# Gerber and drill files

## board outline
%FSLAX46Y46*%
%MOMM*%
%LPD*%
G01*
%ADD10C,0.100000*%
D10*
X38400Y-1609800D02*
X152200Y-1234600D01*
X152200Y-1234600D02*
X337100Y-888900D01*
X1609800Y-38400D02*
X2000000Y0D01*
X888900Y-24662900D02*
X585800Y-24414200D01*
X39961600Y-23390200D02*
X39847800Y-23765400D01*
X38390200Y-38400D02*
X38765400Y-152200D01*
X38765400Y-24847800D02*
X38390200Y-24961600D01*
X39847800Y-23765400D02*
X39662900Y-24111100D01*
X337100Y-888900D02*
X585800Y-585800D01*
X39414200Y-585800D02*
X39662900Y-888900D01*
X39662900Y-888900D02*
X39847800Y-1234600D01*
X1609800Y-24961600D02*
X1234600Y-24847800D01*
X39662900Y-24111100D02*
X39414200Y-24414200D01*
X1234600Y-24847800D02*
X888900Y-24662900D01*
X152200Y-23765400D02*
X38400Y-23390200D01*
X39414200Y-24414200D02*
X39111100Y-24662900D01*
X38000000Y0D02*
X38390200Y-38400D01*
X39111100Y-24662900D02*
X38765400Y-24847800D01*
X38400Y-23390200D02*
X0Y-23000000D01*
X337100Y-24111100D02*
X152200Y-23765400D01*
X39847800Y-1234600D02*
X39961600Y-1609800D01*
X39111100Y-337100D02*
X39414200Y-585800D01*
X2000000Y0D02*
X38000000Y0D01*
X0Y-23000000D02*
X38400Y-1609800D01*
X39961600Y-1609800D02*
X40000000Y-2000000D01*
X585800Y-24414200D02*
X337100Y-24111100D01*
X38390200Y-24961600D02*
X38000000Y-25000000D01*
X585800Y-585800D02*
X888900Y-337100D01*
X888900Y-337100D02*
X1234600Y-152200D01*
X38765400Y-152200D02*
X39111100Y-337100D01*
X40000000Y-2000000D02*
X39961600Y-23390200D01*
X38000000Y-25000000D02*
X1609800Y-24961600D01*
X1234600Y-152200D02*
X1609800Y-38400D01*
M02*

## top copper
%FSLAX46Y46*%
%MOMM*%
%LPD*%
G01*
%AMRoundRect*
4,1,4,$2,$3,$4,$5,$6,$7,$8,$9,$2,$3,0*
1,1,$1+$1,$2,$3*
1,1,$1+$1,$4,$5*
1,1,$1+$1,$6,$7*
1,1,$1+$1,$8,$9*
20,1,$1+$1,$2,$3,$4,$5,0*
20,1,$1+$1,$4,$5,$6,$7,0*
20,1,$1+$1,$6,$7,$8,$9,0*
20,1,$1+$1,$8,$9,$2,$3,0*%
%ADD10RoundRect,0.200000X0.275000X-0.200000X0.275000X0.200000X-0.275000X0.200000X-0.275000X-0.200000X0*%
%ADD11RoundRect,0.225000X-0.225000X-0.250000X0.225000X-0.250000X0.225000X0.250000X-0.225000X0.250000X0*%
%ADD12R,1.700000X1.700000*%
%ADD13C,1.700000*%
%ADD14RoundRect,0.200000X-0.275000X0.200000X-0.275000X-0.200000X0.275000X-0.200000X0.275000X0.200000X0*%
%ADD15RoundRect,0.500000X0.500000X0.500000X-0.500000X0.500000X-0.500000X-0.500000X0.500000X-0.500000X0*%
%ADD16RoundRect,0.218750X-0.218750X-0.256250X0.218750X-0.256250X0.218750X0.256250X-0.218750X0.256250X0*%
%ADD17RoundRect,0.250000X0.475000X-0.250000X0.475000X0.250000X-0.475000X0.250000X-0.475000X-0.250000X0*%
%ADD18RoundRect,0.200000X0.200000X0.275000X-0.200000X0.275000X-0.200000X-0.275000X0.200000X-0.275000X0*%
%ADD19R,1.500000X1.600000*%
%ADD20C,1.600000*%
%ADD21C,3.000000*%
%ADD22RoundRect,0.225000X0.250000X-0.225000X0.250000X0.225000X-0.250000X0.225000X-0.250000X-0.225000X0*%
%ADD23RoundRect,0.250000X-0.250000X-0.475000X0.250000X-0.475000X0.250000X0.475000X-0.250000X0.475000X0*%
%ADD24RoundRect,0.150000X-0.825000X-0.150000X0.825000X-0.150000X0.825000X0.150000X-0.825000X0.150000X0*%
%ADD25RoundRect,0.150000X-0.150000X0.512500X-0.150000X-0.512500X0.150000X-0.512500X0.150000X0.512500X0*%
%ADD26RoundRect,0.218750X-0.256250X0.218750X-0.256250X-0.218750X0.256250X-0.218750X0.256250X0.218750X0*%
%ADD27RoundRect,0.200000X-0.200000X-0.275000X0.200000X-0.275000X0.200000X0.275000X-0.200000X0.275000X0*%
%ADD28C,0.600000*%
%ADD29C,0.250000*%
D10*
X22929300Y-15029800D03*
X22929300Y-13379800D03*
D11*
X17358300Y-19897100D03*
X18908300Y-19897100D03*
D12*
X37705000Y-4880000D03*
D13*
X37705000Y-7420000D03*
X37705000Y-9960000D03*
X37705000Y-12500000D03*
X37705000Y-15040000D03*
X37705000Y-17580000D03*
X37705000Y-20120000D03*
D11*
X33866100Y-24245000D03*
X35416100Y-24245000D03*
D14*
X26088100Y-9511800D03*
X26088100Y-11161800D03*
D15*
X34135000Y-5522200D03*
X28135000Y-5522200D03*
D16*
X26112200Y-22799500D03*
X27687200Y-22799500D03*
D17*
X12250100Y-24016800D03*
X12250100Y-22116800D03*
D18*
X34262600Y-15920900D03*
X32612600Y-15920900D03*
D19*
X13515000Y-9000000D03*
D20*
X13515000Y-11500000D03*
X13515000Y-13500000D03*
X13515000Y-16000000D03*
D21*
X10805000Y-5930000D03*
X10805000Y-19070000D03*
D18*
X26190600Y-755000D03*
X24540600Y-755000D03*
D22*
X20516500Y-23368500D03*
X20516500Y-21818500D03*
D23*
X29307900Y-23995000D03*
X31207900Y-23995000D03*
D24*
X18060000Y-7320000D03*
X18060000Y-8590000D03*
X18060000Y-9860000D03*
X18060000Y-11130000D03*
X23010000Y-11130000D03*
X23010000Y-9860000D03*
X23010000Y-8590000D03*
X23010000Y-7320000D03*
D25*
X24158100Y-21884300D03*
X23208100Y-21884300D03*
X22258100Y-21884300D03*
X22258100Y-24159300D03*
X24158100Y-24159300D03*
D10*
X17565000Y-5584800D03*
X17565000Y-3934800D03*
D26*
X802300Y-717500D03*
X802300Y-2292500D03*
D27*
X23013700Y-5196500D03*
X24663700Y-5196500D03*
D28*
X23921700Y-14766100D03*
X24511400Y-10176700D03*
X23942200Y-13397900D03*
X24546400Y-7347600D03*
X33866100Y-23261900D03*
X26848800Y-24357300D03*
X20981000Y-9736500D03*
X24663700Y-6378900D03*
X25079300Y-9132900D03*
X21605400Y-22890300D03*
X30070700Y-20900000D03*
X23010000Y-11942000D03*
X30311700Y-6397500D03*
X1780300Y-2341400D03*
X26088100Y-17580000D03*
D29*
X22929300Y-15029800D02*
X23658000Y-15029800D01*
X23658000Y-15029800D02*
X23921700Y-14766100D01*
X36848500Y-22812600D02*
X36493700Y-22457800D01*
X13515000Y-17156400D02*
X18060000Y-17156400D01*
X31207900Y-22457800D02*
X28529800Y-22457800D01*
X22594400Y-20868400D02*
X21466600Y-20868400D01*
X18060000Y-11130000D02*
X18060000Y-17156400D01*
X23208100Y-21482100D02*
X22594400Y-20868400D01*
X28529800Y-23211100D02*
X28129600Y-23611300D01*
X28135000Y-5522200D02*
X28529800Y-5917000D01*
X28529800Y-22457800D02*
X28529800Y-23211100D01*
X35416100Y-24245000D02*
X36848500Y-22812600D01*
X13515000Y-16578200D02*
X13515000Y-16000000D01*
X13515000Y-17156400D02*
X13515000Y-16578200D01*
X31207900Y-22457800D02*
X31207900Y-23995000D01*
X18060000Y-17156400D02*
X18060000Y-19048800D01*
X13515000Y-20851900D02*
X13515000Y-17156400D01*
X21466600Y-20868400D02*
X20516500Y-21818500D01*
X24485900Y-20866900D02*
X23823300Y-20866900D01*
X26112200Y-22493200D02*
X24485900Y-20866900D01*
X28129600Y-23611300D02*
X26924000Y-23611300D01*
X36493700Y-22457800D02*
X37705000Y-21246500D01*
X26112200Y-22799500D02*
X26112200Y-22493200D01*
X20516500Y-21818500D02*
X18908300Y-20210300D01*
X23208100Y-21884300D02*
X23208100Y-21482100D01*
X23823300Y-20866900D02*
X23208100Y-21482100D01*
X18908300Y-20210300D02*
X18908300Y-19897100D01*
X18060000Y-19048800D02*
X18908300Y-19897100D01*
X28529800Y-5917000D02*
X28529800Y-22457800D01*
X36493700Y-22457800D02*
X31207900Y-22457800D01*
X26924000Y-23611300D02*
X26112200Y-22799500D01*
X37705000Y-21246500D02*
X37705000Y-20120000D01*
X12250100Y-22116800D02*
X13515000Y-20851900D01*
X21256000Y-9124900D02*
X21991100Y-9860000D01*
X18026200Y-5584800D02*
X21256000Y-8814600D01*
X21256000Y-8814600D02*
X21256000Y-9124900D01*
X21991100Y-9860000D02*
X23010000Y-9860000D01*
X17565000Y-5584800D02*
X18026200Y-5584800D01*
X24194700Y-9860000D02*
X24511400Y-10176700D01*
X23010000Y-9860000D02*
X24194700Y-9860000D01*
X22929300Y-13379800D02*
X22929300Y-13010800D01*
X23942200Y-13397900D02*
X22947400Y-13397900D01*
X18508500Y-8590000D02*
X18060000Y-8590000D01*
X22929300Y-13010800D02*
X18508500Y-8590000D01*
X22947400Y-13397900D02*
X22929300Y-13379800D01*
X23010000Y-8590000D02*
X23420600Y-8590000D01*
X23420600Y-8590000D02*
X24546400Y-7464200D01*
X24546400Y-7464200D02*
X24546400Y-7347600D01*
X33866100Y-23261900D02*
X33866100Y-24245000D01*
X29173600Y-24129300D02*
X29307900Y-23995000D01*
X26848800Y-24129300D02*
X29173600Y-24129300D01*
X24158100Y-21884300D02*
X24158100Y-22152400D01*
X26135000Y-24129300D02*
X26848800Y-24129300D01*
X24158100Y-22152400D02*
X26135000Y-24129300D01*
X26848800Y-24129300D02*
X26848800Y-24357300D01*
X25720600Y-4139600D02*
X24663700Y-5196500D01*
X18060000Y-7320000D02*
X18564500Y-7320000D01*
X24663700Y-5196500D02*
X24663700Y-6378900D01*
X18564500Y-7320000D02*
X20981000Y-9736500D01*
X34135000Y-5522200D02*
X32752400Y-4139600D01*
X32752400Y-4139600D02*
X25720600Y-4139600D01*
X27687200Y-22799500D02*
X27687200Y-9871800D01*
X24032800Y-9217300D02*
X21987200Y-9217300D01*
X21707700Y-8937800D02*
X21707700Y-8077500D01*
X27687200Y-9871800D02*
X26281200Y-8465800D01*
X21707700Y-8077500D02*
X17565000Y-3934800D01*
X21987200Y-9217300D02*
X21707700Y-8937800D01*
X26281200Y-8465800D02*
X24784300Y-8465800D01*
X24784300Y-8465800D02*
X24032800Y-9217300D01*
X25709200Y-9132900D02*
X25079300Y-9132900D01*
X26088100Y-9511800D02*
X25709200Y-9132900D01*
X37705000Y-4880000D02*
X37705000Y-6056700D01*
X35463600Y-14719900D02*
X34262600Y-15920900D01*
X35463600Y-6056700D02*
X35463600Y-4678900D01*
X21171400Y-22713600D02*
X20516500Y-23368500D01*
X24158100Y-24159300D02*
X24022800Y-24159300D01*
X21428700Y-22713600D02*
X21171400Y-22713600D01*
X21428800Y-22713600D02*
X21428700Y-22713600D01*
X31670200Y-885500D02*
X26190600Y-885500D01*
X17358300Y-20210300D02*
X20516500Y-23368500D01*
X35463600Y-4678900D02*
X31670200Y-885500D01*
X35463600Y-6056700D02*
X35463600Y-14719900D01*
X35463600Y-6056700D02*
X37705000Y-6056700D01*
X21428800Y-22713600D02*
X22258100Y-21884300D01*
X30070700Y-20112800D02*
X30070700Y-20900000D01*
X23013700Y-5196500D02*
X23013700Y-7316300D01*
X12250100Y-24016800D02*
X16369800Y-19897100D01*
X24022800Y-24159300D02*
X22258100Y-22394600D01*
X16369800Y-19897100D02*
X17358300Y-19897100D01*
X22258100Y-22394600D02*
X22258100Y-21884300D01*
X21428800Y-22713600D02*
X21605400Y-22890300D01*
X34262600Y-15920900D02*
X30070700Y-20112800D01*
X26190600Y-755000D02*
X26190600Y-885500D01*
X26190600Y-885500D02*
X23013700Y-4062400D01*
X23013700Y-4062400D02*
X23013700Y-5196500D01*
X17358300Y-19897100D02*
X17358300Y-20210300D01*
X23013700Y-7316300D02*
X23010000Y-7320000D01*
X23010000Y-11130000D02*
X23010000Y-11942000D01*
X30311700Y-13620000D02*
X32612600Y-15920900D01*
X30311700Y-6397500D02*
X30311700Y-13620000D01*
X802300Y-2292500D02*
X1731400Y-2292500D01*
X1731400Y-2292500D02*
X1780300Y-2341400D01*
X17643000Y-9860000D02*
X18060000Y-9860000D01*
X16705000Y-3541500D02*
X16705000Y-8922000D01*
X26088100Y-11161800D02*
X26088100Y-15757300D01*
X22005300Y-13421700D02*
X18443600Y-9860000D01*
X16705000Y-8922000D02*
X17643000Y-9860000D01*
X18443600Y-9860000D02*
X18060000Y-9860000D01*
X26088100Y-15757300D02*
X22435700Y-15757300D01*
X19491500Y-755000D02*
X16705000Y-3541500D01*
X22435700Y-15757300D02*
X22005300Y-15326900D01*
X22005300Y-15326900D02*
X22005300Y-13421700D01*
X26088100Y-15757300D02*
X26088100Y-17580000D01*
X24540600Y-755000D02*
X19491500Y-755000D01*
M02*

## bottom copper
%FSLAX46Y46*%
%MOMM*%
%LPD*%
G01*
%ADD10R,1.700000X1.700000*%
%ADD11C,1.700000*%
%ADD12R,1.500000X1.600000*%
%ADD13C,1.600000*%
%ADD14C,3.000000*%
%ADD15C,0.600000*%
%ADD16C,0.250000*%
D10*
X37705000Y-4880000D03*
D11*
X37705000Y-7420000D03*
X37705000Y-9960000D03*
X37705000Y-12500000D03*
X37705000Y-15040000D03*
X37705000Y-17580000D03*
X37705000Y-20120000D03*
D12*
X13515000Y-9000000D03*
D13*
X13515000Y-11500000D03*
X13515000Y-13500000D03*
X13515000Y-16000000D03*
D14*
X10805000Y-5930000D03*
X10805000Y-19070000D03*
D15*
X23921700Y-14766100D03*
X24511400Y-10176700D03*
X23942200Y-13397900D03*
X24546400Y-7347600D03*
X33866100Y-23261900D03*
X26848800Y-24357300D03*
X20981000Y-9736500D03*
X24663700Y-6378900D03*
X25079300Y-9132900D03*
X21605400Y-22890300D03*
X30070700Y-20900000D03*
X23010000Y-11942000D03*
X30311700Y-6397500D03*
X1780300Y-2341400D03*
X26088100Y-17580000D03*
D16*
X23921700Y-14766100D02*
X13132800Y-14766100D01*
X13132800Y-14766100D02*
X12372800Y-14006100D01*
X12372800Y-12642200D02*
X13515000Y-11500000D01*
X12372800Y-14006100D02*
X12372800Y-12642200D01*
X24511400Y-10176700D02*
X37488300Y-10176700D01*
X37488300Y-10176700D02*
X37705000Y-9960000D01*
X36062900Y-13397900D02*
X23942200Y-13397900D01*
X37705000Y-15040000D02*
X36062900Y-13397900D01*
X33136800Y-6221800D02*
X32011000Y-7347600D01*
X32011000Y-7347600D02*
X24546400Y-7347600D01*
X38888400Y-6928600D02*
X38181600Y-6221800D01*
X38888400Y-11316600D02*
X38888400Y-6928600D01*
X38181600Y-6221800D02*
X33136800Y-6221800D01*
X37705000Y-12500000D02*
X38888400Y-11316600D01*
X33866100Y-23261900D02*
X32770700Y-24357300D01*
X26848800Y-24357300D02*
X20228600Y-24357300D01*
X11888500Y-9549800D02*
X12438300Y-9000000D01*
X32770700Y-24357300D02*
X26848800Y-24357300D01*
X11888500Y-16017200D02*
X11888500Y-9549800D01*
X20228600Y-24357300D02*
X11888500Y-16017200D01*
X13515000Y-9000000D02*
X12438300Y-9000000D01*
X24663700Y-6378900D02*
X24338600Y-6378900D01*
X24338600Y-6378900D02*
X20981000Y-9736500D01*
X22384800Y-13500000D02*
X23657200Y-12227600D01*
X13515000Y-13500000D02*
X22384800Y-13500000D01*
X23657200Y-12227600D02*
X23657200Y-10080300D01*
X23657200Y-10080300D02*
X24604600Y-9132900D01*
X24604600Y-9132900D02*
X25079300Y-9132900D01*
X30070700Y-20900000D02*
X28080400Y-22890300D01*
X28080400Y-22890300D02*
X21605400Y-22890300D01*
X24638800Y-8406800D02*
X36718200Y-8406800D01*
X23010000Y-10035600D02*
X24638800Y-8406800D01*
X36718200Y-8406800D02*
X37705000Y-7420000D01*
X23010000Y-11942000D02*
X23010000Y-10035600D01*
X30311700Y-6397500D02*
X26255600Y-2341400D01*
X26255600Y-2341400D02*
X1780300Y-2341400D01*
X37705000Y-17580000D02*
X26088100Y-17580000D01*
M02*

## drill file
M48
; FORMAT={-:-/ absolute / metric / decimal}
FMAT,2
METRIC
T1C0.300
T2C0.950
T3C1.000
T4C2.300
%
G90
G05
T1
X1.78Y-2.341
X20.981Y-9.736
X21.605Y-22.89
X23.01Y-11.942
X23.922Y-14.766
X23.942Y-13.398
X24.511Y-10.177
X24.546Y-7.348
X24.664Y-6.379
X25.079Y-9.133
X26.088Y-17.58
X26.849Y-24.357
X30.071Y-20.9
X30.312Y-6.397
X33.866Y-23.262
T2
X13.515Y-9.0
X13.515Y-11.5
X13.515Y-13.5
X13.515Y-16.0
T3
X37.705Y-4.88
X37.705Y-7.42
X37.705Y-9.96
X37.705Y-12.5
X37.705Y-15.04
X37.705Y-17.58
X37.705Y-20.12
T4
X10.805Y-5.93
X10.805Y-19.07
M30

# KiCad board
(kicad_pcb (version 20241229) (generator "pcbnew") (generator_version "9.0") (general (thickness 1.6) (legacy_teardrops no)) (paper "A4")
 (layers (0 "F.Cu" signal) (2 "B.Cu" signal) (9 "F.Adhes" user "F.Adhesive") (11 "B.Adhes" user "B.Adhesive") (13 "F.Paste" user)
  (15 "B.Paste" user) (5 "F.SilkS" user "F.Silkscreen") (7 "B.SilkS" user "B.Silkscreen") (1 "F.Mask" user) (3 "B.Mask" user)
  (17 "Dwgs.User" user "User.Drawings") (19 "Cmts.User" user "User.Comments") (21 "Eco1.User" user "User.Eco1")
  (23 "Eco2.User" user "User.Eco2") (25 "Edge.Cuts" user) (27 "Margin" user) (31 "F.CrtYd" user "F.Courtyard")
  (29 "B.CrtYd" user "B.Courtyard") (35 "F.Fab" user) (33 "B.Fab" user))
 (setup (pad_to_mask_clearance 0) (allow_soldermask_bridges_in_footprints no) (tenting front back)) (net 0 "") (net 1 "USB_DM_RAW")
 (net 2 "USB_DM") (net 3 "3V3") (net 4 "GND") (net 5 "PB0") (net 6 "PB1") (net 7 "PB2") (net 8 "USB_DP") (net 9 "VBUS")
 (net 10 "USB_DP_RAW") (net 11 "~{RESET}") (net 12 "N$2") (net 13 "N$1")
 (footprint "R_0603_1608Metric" (layer "F.Cu") (at 22.9293 14.2048 90)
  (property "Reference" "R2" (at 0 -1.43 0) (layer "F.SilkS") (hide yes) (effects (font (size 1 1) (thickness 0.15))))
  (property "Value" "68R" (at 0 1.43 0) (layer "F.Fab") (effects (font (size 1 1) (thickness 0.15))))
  (pad "1" smd roundrect (at -0.825 0 90) (size 0.8 0.95) (layers "F.Cu" "F.Mask" "F.Paste") (roundrect_rratio 0.25) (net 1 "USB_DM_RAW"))
  (pad "2" smd roundrect (at 0.825 0 90) (size 0.8 0.95) (layers "F.Cu" "F.Mask" "F.Paste") (roundrect_rratio 0.25) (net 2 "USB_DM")))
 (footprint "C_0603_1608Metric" (layer "F.Cu") (at 18.1333 19.8971)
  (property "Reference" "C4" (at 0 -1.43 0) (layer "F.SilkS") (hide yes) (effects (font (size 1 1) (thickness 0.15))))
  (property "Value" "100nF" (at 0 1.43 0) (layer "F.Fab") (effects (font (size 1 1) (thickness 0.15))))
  (pad "1" smd roundrect (at -0.775 0) (size 0.9 0.95) (layers "F.Cu" "F.Mask" "F.Paste") (roundrect_rratio 0.25) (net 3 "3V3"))
  (pad "2" smd roundrect (at 0.775 0) (size 0.9 0.95) (layers "F.Cu" "F.Mask" "F.Paste") (roundrect_rratio 0.25) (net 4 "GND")))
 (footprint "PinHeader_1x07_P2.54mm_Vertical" (layer "F.Cu") (at 37.705 4.88)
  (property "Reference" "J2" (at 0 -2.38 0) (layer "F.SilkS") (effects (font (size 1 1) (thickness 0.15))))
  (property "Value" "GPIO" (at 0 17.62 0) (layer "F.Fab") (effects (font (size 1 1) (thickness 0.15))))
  (pad "1" thru_hole rect (at 0 0) (size 1.7 1.7) (drill 1) (layers "*.Cu" "*.Mask") (remove_unused_layers no) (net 3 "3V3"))
  (pad "2" thru_hole circle (at 0 2.54) (size 1.7 1.7) (drill 1) (layers "*.Cu" "*.Mask") (remove_unused_layers no) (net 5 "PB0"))
  (pad "3" thru_hole circle (at 0 5.08) (size 1.7 1.7) (drill 1) (layers "*.Cu" "*.Mask") (remove_unused_layers no) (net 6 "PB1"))
  (pad "4" thru_hole circle (at 0 7.62) (size 1.7 1.7) (drill 1) (layers "*.Cu" "*.Mask") (remove_unused_layers no) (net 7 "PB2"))
  (pad "5" thru_hole circle (at 0 10.16) (size 1.7 1.7) (drill 1) (layers "*.Cu" "*.Mask") (remove_unused_layers no) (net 2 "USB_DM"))
  (pad "6" thru_hole circle (at 0 12.7) (size 1.7 1.7) (drill 1) (layers "*.Cu" "*.Mask") (remove_unused_layers no) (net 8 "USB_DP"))
  (pad "7" thru_hole circle (at 0 15.24) (size 1.7 1.7) (drill 1) (layers "*.Cu" "*.Mask") (remove_unused_layers no) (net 4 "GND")))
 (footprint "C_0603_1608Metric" (layer "F.Cu") (at 34.6411 24.245)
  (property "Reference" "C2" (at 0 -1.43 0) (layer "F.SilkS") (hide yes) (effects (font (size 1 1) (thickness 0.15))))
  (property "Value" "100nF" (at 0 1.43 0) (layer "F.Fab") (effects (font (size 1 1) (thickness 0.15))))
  (pad "1" smd roundrect (at -0.775 0) (size 0.9 0.95) (layers "F.Cu" "F.Mask" "F.Paste") (roundrect_rratio 0.25) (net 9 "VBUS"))
  (pad "2" smd roundrect (at 0.775 0) (size 0.9 0.95) (layers "F.Cu" "F.Mask" "F.Paste") (roundrect_rratio 0.25) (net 4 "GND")))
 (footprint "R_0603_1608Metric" (layer "F.Cu") (at 26.0881 10.3368 -90)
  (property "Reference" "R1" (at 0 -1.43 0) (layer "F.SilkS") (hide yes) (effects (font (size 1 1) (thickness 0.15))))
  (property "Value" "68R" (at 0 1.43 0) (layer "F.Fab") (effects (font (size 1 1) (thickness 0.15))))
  (pad "1" smd roundrect (at -0.825 0 270) (size 0.8 0.95) (layers "F.Cu" "F.Mask" "F.Paste") (roundrect_rratio 0.25) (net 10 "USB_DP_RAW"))
  (pad "2" smd roundrect (at 0.825 0 270) (size 0.8 0.95) (layers "F.Cu" "F.Mask" "F.Paste") (roundrect_rratio 0.25) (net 8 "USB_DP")))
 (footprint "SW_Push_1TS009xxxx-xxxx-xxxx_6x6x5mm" (layer "F.Cu") (at 31.135 5.5222 180)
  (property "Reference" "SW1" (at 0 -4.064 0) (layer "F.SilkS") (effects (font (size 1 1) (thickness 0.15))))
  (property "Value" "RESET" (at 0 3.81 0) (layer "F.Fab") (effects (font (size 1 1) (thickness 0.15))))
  (pad "1" smd roundrect (at -3 0 180) (size 2 2) (layers "F.Cu" "F.Mask" "F.Paste") (roundrect_rratio 0.25) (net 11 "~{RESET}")
   (thermal_bridge_angle 45))
  (pad "2" smd roundrect (at 3 0 180) (size 2 2) (layers "F.Cu" "F.Mask" "F.Paste") (roundrect_rratio 0.25) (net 4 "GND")
   (thermal_bridge_angle 45)))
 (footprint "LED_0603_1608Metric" (layer "F.Cu") (at 26.8997 22.7995)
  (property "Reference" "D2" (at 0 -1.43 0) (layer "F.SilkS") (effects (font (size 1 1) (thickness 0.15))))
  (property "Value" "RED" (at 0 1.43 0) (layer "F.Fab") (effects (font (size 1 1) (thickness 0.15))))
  (pad "1" smd roundrect (at -0.7875 0) (size 0.875 0.95) (layers "F.Cu" "F.Mask" "F.Paste") (roundrect_rratio 0.25) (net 4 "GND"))
  (pad "2" smd roundrect (at 0.7875 0) (size 0.875 0.95) (layers "F.Cu" "F.Mask" "F.Paste") (roundrect_rratio 0.25) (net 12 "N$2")))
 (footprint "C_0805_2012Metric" (layer "F.Cu") (at 12.2501 23.0668 90)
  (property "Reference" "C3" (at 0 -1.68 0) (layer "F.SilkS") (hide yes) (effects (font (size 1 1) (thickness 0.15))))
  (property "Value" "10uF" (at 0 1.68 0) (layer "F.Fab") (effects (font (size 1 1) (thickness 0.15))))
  (pad "1" smd roundrect (at -0.95 0 90) (size 1 1.45) (layers "F.Cu" "F.Mask" "F.Paste") (roundrect_rratio 0.25) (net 3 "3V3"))
  (pad "2" smd roundrect (at 0.95 0 90) (size 1 1.45) (layers "F.Cu" "F.Mask" "F.Paste") (roundrect_rratio 0.25) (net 4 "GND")))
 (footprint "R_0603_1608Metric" (layer "F.Cu") (at 33.4376 15.9209 180)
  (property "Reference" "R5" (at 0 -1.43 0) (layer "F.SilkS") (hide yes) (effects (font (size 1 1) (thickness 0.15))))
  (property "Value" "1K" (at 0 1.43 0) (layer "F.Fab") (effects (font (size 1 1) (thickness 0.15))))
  (pad "1" smd roundrect (at -0.825 0 180) (size 0.8 0.95) (layers "F.Cu" "F.Mask" "F.Paste") (roundrect_rratio 0.25) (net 3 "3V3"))
  (pad "2" smd roundrect (at 0.825 0 180) (size 0.8 0.95) (layers "F.Cu" "F.Mask" "F.Paste") (roundrect_rratio 0.25) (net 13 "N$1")))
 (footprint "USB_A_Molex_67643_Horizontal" (layer "F.Cu") (at 13.515 9 -90)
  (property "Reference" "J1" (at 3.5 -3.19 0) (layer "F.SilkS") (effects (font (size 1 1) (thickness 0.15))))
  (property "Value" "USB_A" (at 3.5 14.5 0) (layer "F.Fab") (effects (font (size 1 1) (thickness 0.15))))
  (pad "1" thru_hole rect (at 0 0 270) (size 1.6 1.5) (drill 0.95) (layers "*.Cu" "*.Mask") (remove_unused_layers no) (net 9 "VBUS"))
  (pad "2" thru_hole circle (at 2.5 0 270) (size 1.6 1.6) (drill 0.95) (layers "*.Cu" "*.Mask") (remove_unused_layers no)
   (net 1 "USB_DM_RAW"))
  (pad "3" thru_hole circle (at 4.5 0 270) (size 1.6 1.6) (drill 0.95) (layers "*.Cu" "*.Mask") (remove_unused_layers no)
   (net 10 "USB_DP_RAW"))
  (pad "4" thru_hole circle (at 7 0 270) (size 1.6 1.6) (drill 0.95) (layers "*.Cu" "*.Mask") (remove_unused_layers no) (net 4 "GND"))
  (pad "5" thru_hole circle (at -3.07 2.71 270) (size 3 3) (drill 2.3) (layers "*.Cu" "*.Mask") (remove_unused_layers no))
  (pad "5" thru_hole circle (at 10.07 2.71 270) (size 3 3) (drill 2.3) (layers "*.Cu" "*.Mask") (remove_unused_layers no)))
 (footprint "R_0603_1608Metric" (layer "F.Cu") (at 25.3656 0.755 180)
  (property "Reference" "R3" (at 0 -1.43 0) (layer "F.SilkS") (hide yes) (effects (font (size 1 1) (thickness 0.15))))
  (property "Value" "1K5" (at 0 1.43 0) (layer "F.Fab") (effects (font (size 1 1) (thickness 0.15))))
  (pad "1" smd roundrect (at -0.825 0 180) (size 0.8 0.95) (layers "F.Cu" "F.Mask" "F.Paste") (roundrect_rratio 0.25) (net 3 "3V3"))
  (pad "2" smd roundrect (at 0.825 0 180) (size 0.8 0.95) (layers "F.Cu" "F.Mask" "F.Paste") (roundrect_rratio 0.25) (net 8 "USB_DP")))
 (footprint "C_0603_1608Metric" (layer "F.Cu") (at 20.5165 22.5935 90)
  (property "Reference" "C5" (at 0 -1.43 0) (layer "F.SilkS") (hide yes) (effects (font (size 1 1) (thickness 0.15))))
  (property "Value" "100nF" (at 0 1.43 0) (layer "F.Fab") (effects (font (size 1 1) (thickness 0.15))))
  (pad "1" smd roundrect (at -0.775 0 90) (size 0.9 0.95) (layers "F.Cu" "F.Mask" "F.Paste") (roundrect_rratio 0.25) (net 3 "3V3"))
  (pad "2" smd roundrect (at 0.775 0 90) (size 0.9 0.95) (layers "F.Cu" "F.Mask" "F.Paste") (roundrect_rratio 0.25) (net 4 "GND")))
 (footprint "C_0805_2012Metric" (layer "F.Cu") (at 30.2579 23.995)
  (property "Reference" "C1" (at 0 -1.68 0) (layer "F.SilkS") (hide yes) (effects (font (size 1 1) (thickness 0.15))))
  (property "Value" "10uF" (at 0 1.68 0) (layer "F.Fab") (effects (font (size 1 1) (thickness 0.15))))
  (pad "1" smd roundrect (at -0.95 0) (size 1 1.45) (layers "F.Cu" "F.Mask" "F.Paste") (roundrect_rratio 0.25) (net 9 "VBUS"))
  (pad "2" smd roundrect (at 0.95 0) (size 1 1.45) (layers "F.Cu" "F.Mask" "F.Paste") (roundrect_rratio 0.25) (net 4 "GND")))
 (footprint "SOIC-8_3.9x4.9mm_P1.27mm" (layer "F.Cu") (at 20.535 9.225)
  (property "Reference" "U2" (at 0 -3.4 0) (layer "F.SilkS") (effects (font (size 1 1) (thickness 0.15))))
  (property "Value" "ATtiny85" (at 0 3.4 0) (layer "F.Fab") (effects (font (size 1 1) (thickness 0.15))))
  (pad "1" smd roundrect (at -2.475 -1.905) (size 1.95 0.6) (layers "F.Cu" "F.Mask" "F.Paste") (roundrect_rratio 0.25) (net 11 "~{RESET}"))
  (pad "2" smd roundrect (at -2.475 -0.635) (size 1.95 0.6) (layers "F.Cu" "F.Mask" "F.Paste") (roundrect_rratio 0.25) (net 2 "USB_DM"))
  (pad "3" smd roundrect (at -2.475 0.635) (size 1.95 0.6) (layers "F.Cu" "F.Mask" "F.Paste") (roundrect_rratio 0.25) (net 8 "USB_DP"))
  (pad "4" smd roundrect (at -2.475 1.905) (size 1.95 0.6) (layers "F.Cu" "F.Mask" "F.Paste") (roundrect_rratio 0.25) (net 4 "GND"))
  (pad "5" smd roundrect (at 2.475 1.905) (size 1.95 0.6) (layers "F.Cu" "F.Mask" "F.Paste") (roundrect_rratio 0.25) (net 5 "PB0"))
  (pad "6" smd roundrect (at 2.475 0.635) (size 1.95 0.6) (layers "F.Cu" "F.Mask" "F.Paste") (roundrect_rratio 0.25) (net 6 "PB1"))
  (pad "7" smd roundrect (at 2.475 -0.635) (size 1.95 0.6) (layers "F.Cu" "F.Mask" "F.Paste") (roundrect_rratio 0.25) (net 7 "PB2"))
  (pad "8" smd roundrect (at 2.475 -1.905) (size 1.95 0.6) (layers "F.Cu" "F.Mask" "F.Paste") (roundrect_rratio 0.25) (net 3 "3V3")))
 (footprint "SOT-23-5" (layer "F.Cu") (at 23.2081 23.0218 -90)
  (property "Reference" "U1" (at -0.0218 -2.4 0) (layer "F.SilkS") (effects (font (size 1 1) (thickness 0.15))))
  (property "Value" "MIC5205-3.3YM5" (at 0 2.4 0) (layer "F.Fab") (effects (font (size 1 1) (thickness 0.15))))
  (pad "1" smd roundrect (at -1.1375 -0.95 270) (size 1.325 0.6) (layers "F.Cu" "F.Mask" "F.Paste") (roundrect_rratio 0.25) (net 9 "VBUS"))
  (pad "2" smd roundrect (at -1.1375 0 270) (size 1.325 0.6) (layers "F.Cu" "F.Mask" "F.Paste") (roundrect_rratio 0.25) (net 4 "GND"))
  (pad "3" smd roundrect (at -1.1375 0.95 270) (size 1.325 0.6) (layers "F.Cu" "F.Mask" "F.Paste") (roundrect_rratio 0.25) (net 3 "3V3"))
  (pad "4" smd roundrect (at 1.1375 0.95 270) (size 1.325 0.6) (layers "F.Cu" "F.Mask" "F.Paste") (roundrect_rratio 0.25))
  (pad "5" smd roundrect (at 1.1375 -0.95 270) (size 1.325 0.6) (layers "F.Cu" "F.Mask" "F.Paste") (roundrect_rratio 0.25) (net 3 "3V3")))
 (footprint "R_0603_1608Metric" (layer "F.Cu") (at 17.565 4.7598 90)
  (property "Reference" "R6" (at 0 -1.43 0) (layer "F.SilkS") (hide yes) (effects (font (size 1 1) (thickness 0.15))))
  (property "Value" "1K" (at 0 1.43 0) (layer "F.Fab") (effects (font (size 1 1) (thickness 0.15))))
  (pad "1" smd roundrect (at -0.825 0 90) (size 0.8 0.95) (layers "F.Cu" "F.Mask" "F.Paste") (roundrect_rratio 0.25) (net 6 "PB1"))
  (pad "2" smd roundrect (at 0.825 0 90) (size 0.8 0.95) (layers "F.Cu" "F.Mask" "F.Paste") (roundrect_rratio 0.25) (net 12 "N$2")))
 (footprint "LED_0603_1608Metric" (layer "F.Cu") (at 0.8023 1.505 -90)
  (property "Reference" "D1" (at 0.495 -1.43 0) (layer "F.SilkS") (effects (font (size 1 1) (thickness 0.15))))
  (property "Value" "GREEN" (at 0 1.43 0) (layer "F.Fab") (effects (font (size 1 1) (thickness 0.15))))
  (pad "1" smd roundrect (at -0.7875 0 270) (size 0.875 0.95) (layers "F.Cu" "F.Mask" "F.Paste") (roundrect_rratio 0.25) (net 4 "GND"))
  (pad "2" smd roundrect (at 0.7875 0 270) (size 0.875 0.95) (layers "F.Cu" "F.Mask" "F.Paste") (roundrect_rratio 0.25) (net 13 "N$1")))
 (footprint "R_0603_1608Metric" (layer "F.Cu") (at 23.8387 5.1965)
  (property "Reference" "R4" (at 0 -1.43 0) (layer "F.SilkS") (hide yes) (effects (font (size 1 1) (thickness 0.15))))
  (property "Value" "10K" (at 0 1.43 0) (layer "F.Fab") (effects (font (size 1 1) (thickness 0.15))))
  (pad "1" smd roundrect (at -0.825 0) (size 0.8 0.95) (layers "F.Cu" "F.Mask" "F.Paste") (roundrect_rratio 0.25) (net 3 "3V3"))
  (pad "2" smd roundrect (at 0.825 0) (size 0.8 0.95) (layers "F.Cu" "F.Mask" "F.Paste") (roundrect_rratio 0.25) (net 11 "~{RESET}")))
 (gr_line (start 0.0384 1.6098) (end 0.1522 1.2346) (stroke (width 0.1) (type solid)) (layer "Edge.Cuts"))
 (gr_line (start 0.1522 1.2346) (end 0.3371 0.8889) (stroke (width 0.1) (type solid)) (layer "Edge.Cuts"))
 (gr_line (start 1.6098 0.0384) (end 2 0) (stroke (width 0.1) (type solid)) (layer "Edge.Cuts"))
 (gr_line (start 0.8889 24.6629) (end 0.5858 24.4142) (stroke (width 0.1) (type solid)) (layer "Edge.Cuts"))
 (gr_line (start 39.9616 23.3902) (end 39.8478 23.7654) (stroke (width 0.1) (type solid)) (layer "Edge.Cuts"))
 (gr_line (start 38.3902 0.0384) (end 38.7654 0.1522) (stroke (width 0.1) (type solid)) (layer "Edge.Cuts"))
 (gr_line (start 38.7654 24.8478) (end 38.3902 24.9616) (stroke (width 0.1) (type solid)) (layer "Edge.Cuts"))
 (gr_line (start 39.8478 23.7654) (end 39.6629 24.1111) (stroke (width 0.1) (type solid)) (layer "Edge.Cuts"))
 (gr_line (start 0.3371 0.8889) (end 0.5858 0.5858) (stroke (width 0.1) (type solid)) (layer "Edge.Cuts"))
 (gr_line (start 39.4142 0.5858) (end 39.6629 0.8889) (stroke (width 0.1) (type solid)) (layer "Edge.Cuts"))
 (gr_line (start 39.6629 0.8889) (end 39.8478 1.2346) (stroke (width 0.1) (type solid)) (layer "Edge.Cuts"))
 (gr_line (start 1.6098 24.9616) (end 1.2346 24.8478) (stroke (width 0.1) (type solid)) (layer "Edge.Cuts"))
 (gr_line (start 39.6629 24.1111) (end 39.4142 24.4142) (stroke (width 0.1) (type solid)) (layer "Edge.Cuts"))
 (gr_line (start 1.2346 24.8478) (end 0.8889 24.6629) (stroke (width 0.1) (type solid)) (layer "Edge.Cuts"))
 (gr_line (start 0.1522 23.7654) (end 0.0384 23.3902) (stroke (width 0.1) (type solid)) (layer "Edge.Cuts"))
 (gr_line (start 39.4142 24.4142) (end 39.1111 24.6629) (stroke (width 0.1) (type solid)) (layer "Edge.Cuts"))
 (gr_line (start 38 0) (end 38.3902 0.0384) (stroke (width 0.1) (type solid)) (layer "Edge.Cuts"))
 (gr_line (start 39.1111 24.6629) (end 38.7654 24.8478) (stroke (width 0.1) (type solid)) (layer "Edge.Cuts"))
 (gr_line (start 0.0384 23.3902) (end 0 23) (stroke (width 0.1) (type solid)) (layer "Edge.Cuts"))
 (gr_line (start 0.3371 24.1111) (end 0.1522 23.7654) (stroke (width 0.1) (type solid)) (layer "Edge.Cuts"))
 (gr_line (start 39.8478 1.2346) (end 39.9616 1.6098) (stroke (width 0.1) (type solid)) (layer "Edge.Cuts"))
 (gr_line (start 39.1111 0.3371) (end 39.4142 0.5858) (stroke (width 0.1) (type solid)) (layer "Edge.Cuts"))
 (gr_line (start 2 0) (end 38 0) (stroke (width 0.1) (type solid)) (layer "Edge.Cuts"))
 (gr_line (start 0 23) (end 0.0384 1.6098) (stroke (width 0.1) (type solid)) (layer "Edge.Cuts"))
 (gr_line (start 39.9616 1.6098) (end 40 2) (stroke (width 0.1) (type solid)) (layer "Edge.Cuts"))
 (gr_line (start 0.5858 24.4142) (end 0.3371 24.1111) (stroke (width 0.1) (type solid)) (layer "Edge.Cuts"))
 (gr_line (start 38.3902 24.9616) (end 38 25) (stroke (width 0.1) (type solid)) (layer "Edge.Cuts"))
 (gr_line (start 0.5858 0.5858) (end 0.8889 0.3371) (stroke (width 0.1) (type solid)) (layer "Edge.Cuts"))
 (gr_line (start 0.8889 0.3371) (end 1.2346 0.1522) (stroke (width 0.1) (type solid)) (layer "Edge.Cuts"))
 (gr_line (start 38.7654 0.1522) (end 39.1111 0.3371) (stroke (width 0.1) (type solid)) (layer "Edge.Cuts"))
 (gr_line (start 40 2) (end 39.9616 23.3902) (stroke (width 0.1) (type solid)) (layer "Edge.Cuts"))
 (gr_line (start 38 25) (end 1.6098 24.9616) (stroke (width 0.1) (type solid)) (layer "Edge.Cuts"))
 (gr_line (start 1.2346 0.1522) (end 1.6098 0.0384) (stroke (width 0.1) (type solid)) (layer "Edge.Cuts"))
 (segment (start 22.9293 15.0298) (end 23.658 15.0298) (width 0.25) (layer "F.Cu") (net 1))
 (segment (start 23.658 15.0298) (end 23.9217 14.7661) (width 0.25) (layer "F.Cu") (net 1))
 (via (at 23.9217 14.7661) (size 0.6) (drill 0.3) (layers "F.Cu" "B.Cu") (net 1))
 (segment (start 23.9217 14.7661) (end 13.1328 14.7661) (width 0.25) (layer "B.Cu") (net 1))
 (segment (start 13.1328 14.7661) (end 12.3728 14.0061) (width 0.25) (layer "B.Cu") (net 1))
 (segment (start 12.3728 12.6422) (end 13.515 11.5) (width 0.25) (layer "B.Cu") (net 1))
 (segment (start 12.3728 14.0061) (end 12.3728 12.6422) (width 0.25) (layer "B.Cu") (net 1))
 (segment (start 36.8485 22.8126) (end 36.4937 22.4578) (width 0.25) (layer "F.Cu") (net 4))
 (segment (start 13.515 17.1564) (end 18.06 17.1564) (width 0.25) (layer "F.Cu") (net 4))
 (segment (start 31.2079 22.4578) (end 28.5298 22.4578) (width 0.25) (layer "F.Cu") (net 4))
 (segment (start 22.5944 20.8684) (end 21.4666 20.8684) (width 0.25) (layer "F.Cu") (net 4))
 (segment (start 18.06 11.13) (end 18.06 17.1564) (width 0.25) (layer "F.Cu") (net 4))
 (segment (start 23.2081 21.4821) (end 22.5944 20.8684) (width 0.25) (layer "F.Cu") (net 4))
 (segment (start 28.5298 23.2111) (end 28.1296 23.6113) (width 0.25) (layer "F.Cu") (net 4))
 (segment (start 28.135 5.5222) (end 28.5298 5.917) (width 0.25) (layer "F.Cu") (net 4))
 (segment (start 28.5298 22.4578) (end 28.5298 23.2111) (width 0.25) (layer "F.Cu") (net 4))
 (segment (start 35.4161 24.245) (end 36.8485 22.8126) (width 0.25) (layer "F.Cu") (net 4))
 (segment (start 13.515 16.5782) (end 13.515 16) (width 0.25) (layer "F.Cu") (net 4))
 (segment (start 13.515 17.1564) (end 13.515 16.5782) (width 0.25) (layer "F.Cu") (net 4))
 (segment (start 31.2079 22.4578) (end 31.2079 23.995) (width 0.25) (layer "F.Cu") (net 4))
 (segment (start 18.06 17.1564) (end 18.06 19.0488) (width 0.25) (layer "F.Cu") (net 4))
 (segment (start 13.515 20.8519) (end 13.515 17.1564) (width 0.25) (layer "F.Cu") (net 4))
 (segment (start 21.4666 20.8684) (end 20.5165 21.8185) (width 0.25) (layer "F.Cu") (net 4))
 (segment (start 24.4859 20.8669) (end 23.8233 20.8669) (width 0.25) (layer "F.Cu") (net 4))
 (segment (start 26.1122 22.4932) (end 24.4859 20.8669) (width 0.25) (layer "F.Cu") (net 4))
 (segment (start 28.1296 23.6113) (end 26.924 23.6113) (width 0.25) (layer "F.Cu") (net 4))
 (segment (start 36.4937 22.4578) (end 37.705 21.2465) (width 0.25) (layer "F.Cu") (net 4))
 (segment (start 26.1122 22.7995) (end 26.1122 22.4932) (width 0.25) (layer "F.Cu") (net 4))
 (segment (start 20.5165 21.8185) (end 18.9083 20.2103) (width 0.25) (layer "F.Cu") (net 4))
 (segment (start 23.2081 21.8843) (end 23.2081 21.4821) (width 0.25) (layer "F.Cu") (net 4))
 (segment (start 23.8233 20.8669) (end 23.2081 21.4821) (width 0.25) (layer "F.Cu") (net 4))
 (segment (start 18.9083 20.2103) (end 18.9083 19.8971) (width 0.25) (layer "F.Cu") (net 4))
 (segment (start 18.06 19.0488) (end 18.9083 19.8971) (width 0.25) (layer "F.Cu") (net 4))
 (segment (start 28.5298 5.917) (end 28.5298 22.4578) (width 0.25) (layer "F.Cu") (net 4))
 (segment (start 36.4937 22.4578) (end 31.2079 22.4578) (width 0.25) (layer "F.Cu") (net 4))
 (segment (start 26.924 23.6113) (end 26.1122 22.7995) (width 0.25) (layer "F.Cu") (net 4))
 (segment (start 37.705 21.2465) (end 37.705 20.12) (width 0.25) (layer "F.Cu") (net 4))
 (segment (start 12.2501 22.1168) (end 13.515 20.8519) (width 0.25) (layer "F.Cu") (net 4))
 (segment (start 21.256 9.1249) (end 21.9911 9.86) (width 0.25) (layer "F.Cu") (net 6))
 (segment (start 18.0262 5.5848) (end 21.256 8.8146) (width 0.25) (layer "F.Cu") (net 6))
 (segment (start 21.256 8.8146) (end 21.256 9.1249) (width 0.25) (layer "F.Cu") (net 6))
 (segment (start 21.9911 9.86) (end 23.01 9.86) (width 0.25) (layer "F.Cu") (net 6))
 (segment (start 17.565 5.5848) (end 18.0262 5.5848) (width 0.25) (layer "F.Cu") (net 6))
 (segment (start 24.1947 9.86) (end 24.5114 10.1767) (width 0.25) (layer "F.Cu") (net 6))
 (segment (start 23.01 9.86) (end 24.1947 9.86) (width 0.25) (layer "F.Cu") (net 6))
 (via (at 24.5114 10.1767) (size 0.6) (drill 0.3) (layers "F.Cu" "B.Cu") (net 6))
 (segment (start 24.5114 10.1767) (end 37.4883 10.1767) (width 0.25) (layer "B.Cu") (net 6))
 (segment (start 37.4883 10.1767) (end 37.705 9.96) (width 0.25) (layer "B.Cu") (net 6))
 (segment (start 22.9293 13.3798) (end 22.9293 13.0108) (width 0.25) (layer "F.Cu") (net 2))
 (segment (start 23.9422 13.3979) (end 22.9474 13.3979) (width 0.25) (layer "F.Cu") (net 2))
 (segment (start 18.5085 8.59) (end 18.06 8.59) (width 0.25) (layer "F.Cu") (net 2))
 (segment (start 22.9293 13.0108) (end 18.5085 8.59) (width 0.25) (layer "F.Cu") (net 2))
 (segment (start 22.9474 13.3979) (end 22.9293 13.3798) (width 0.25) (layer "F.Cu") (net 2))
 (via (at 23.9422 13.3979) (size 0.6) (drill 0.3) (layers "F.Cu" "B.Cu") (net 2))
 (segment (start 36.0629 13.3979) (end 23.9422 13.3979) (width 0.25) (layer "B.Cu") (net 2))
 (segment (start 37.705 15.04) (end 36.0629 13.3979) (width 0.25) (layer "B.Cu") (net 2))
 (segment (start 23.01 8.59) (end 23.4206 8.59) (width 0.25) (layer "F.Cu") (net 7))
 (segment (start 23.4206 8.59) (end 24.5464 7.4642) (width 0.25) (layer "F.Cu") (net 7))
 (segment (start 24.5464 7.4642) (end 24.5464 7.3476) (width 0.25) (layer "F.Cu") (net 7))
 (via (at 24.5464 7.3476) (size 0.6) (drill 0.3) (layers "F.Cu" "B.Cu") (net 7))
 (segment (start 33.1368 6.2218) (end 32.011 7.3476) (width 0.25) (layer "B.Cu") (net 7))
 (segment (start 32.011 7.3476) (end 24.5464 7.3476) (width 0.25) (layer "B.Cu") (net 7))
 (segment (start 38.8884 6.9286) (end 38.1816 6.2218) (width 0.25) (layer "B.Cu") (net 7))
 (segment (start 38.8884 11.3166) (end 38.8884 6.9286) (width 0.25) (layer "B.Cu") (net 7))
 (segment (start 38.1816 6.2218) (end 33.1368 6.2218) (width 0.25) (layer "B.Cu") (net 7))
 (segment (start 37.705 12.5) (end 38.8884 11.3166) (width 0.25) (layer "B.Cu") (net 7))
 (segment (start 33.8661 23.2619) (end 33.8661 24.245) (width 0.25) (layer "F.Cu") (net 9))
 (segment (start 29.1736 24.1293) (end 29.3079 23.995) (width 0.25) (layer "F.Cu") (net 9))
 (segment (start 26.8488 24.1293) (end 29.1736 24.1293) (width 0.25) (layer "F.Cu") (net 9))
 (segment (start 24.1581 21.8843) (end 24.1581 22.1524) (width 0.25) (layer "F.Cu") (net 9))
 (segment (start 26.135 24.1293) (end 26.8488 24.1293) (width 0.25) (layer "F.Cu") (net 9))
 (segment (start 24.1581 22.1524) (end 26.135 24.1293) (width 0.25) (layer "F.Cu") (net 9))
 (segment (start 26.8488 24.1293) (end 26.8488 24.3573) (width 0.25) (layer "F.Cu") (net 9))
 (via (at 33.8661 23.2619) (size 0.6) (drill 0.3) (layers "F.Cu" "B.Cu") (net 9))
 (via (at 26.8488 24.3573) (size 0.6) (drill 0.3) (layers "F.Cu" "B.Cu") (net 9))
 (segment (start 33.8661 23.2619) (end 32.7707 24.3573) (width 0.25) (layer "B.Cu") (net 9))
 (segment (start 26.8488 24.3573) (end 20.2286 24.3573) (width 0.25) (layer "B.Cu") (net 9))
 (segment (start 11.8885 9.5498) (end 12.4383 9) (width 0.25) (layer "B.Cu") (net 9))
 (segment (start 32.7707 24.3573) (end 26.8488 24.3573) (width 0.25) (layer "B.Cu") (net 9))
 (segment (start 11.8885 16.0172) (end 11.8885 9.5498) (width 0.25) (layer "B.Cu") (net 9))
 (segment (start 20.2286 24.3573) (end 11.8885 16.0172) (width 0.25) (layer "B.Cu") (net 9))
 (segment (start 13.515 9) (end 12.4383 9) (width 0.25) (layer "B.Cu") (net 9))
 (segment (start 25.7206 4.1396) (end 24.6637 5.1965) (width 0.25) (layer "F.Cu") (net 11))
 (segment (start 18.06 7.32) (end 18.5645 7.32) (width 0.25) (layer "F.Cu") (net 11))
 (segment (start 24.6637 5.1965) (end 24.6637 6.3789) (width 0.25) (layer "F.Cu") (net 11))
 (segment (start 18.5645 7.32) (end 20.981 9.7365) (width 0.25) (layer "F.Cu") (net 11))
 (segment (start 34.135 5.5222) (end 32.7524 4.1396) (width 0.25) (layer "F.Cu") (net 11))
 (segment (start 32.7524 4.1396) (end 25.7206 4.1396) (width 0.25) (layer "F.Cu") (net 11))
 (via (at 20.981 9.7365) (size 0.6) (drill 0.3) (layers "F.Cu" "B.Cu") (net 11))
 (via (at 24.6637 6.3789) (size 0.6) (drill 0.3) (layers "F.Cu" "B.Cu") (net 11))
 (segment (start 24.6637 6.3789) (end 24.3386 6.3789) (width 0.25) (layer "B.Cu") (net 11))
 (segment (start 24.3386 6.3789) (end 20.981 9.7365) (width 0.25) (layer "B.Cu") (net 11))
 (segment (start 27.6872 22.7995) (end 27.6872 9.8718) (width 0.25) (layer "F.Cu") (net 12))
 (segment (start 24.0328 9.2173) (end 21.9872 9.2173) (width 0.25) (layer "F.Cu") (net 12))
 (segment (start 21.7077 8.9378) (end 21.7077 8.0775) (width 0.25) (layer "F.Cu") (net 12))
 (segment (start 27.6872 9.8718) (end 26.2812 8.4658) (width 0.25) (layer "F.Cu") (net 12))
 (segment (start 21.7077 8.0775) (end 17.565 3.9348) (width 0.25) (layer "F.Cu") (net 12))
 (segment (start 21.9872 9.2173) (end 21.7077 8.9378) (width 0.25) (layer "F.Cu") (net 12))
 (segment (start 26.2812 8.4658) (end 24.7843 8.4658) (width 0.25) (layer "F.Cu") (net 12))
 (segment (start 24.7843 8.4658) (end 24.0328 9.2173) (width 0.25) (layer "F.Cu") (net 12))
 (segment (start 25.7092 9.1329) (end 25.0793 9.1329) (width 0.25) (layer "F.Cu") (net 10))
 (segment (start 26.0881 9.5118) (end 25.7092 9.1329) (width 0.25) (layer "F.Cu") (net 10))
 (via (at 25.0793 9.1329) (size 0.6) (drill 0.3) (layers "F.Cu" "B.Cu") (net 10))
 (segment (start 22.3848 13.5) (end 23.6572 12.2276) (width 0.25) (layer "B.Cu") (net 10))
 (segment (start 13.515 13.5) (end 22.3848 13.5) (width 0.25) (layer "B.Cu") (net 10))
 (segment (start 23.6572 12.2276) (end 23.6572 10.0803) (width 0.25) (layer "B.Cu") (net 10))
 (segment (start 23.6572 10.0803) (end 24.6046 9.1329) (width 0.25) (layer "B.Cu") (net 10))
 (segment (start 24.6046 9.1329) (end 25.0793 9.1329) (width 0.25) (layer "B.Cu") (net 10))
 (segment (start 37.705 4.88) (end 37.705 6.0567) (width 0.25) (layer "F.Cu") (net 3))
 (segment (start 35.4636 14.7199) (end 34.2626 15.9209) (width 0.25) (layer "F.Cu") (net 3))
 (segment (start 35.4636 6.0567) (end 35.4636 4.6789) (width 0.25) (layer "F.Cu") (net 3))
 (segment (start 21.1714 22.7136) (end 20.5165 23.3685) (width 0.25) (layer "F.Cu") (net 3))
 (segment (start 24.1581 24.1593) (end 24.0228 24.1593) (width 0.25) (layer "F.Cu") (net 3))
 (segment (start 21.4287 22.7136) (end 21.1714 22.7136) (width 0.25) (layer "F.Cu") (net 3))
 (segment (start 21.4288 22.7136) (end 21.4287 22.7136) (width 0.25) (layer "F.Cu") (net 3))
 (segment (start 31.6702 0.8855) (end 26.1906 0.8855) (width 0.25) (layer "F.Cu") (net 3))
 (segment (start 17.3583 20.2103) (end 20.5165 23.3685) (width 0.25) (layer "F.Cu") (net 3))
 (segment (start 35.4636 4.6789) (end 31.6702 0.8855) (width 0.25) (layer "F.Cu") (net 3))
 (segment (start 35.4636 6.0567) (end 35.4636 14.7199) (width 0.25) (layer "F.Cu") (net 3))
 (segment (start 35.4636 6.0567) (end 37.705 6.0567) (width 0.25) (layer "F.Cu") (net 3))
 (segment (start 21.4288 22.7136) (end 22.2581 21.8843) (width 0.25) (layer "F.Cu") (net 3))
 (segment (start 30.0707 20.1128) (end 30.0707 20.9) (width 0.25) (layer "F.Cu") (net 3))
 (segment (start 23.0137 5.1965) (end 23.0137 7.3163) (width 0.25) (layer "F.Cu") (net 3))
 (segment (start 12.2501 24.0168) (end 16.3698 19.8971) (width 0.25) (layer "F.Cu") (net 3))
 (segment (start 24.0228 24.1593) (end 22.2581 22.3946) (width 0.25) (layer "F.Cu") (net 3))
 (segment (start 16.3698 19.8971) (end 17.3583 19.8971) (width 0.25) (layer "F.Cu") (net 3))
 (segment (start 22.2581 22.3946) (end 22.2581 21.8843) (width 0.25) (layer "F.Cu") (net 3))
 (segment (start 21.4288 22.7136) (end 21.6054 22.8903) (width 0.25) (layer "F.Cu") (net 3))
 (segment (start 34.2626 15.9209) (end 30.0707 20.1128) (width 0.25) (layer "F.Cu") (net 3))
 (segment (start 26.1906 0.755) (end 26.1906 0.8855) (width 0.25) (layer "F.Cu") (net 3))
 (segment (start 26.1906 0.8855) (end 23.0137 4.0624) (width 0.25) (layer "F.Cu") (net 3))
 (segment (start 23.0137 4.0624) (end 23.0137 5.1965) (width 0.25) (layer "F.Cu") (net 3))
 (segment (start 17.3583 19.8971) (end 17.3583 20.2103) (width 0.25) (layer "F.Cu") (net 3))
 (segment (start 23.0137 7.3163) (end 23.01 7.32) (width 0.25) (layer "F.Cu") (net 3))
 (via (at 21.6054 22.8903) (size 0.6) (drill 0.3) (layers "F.Cu" "B.Cu") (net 3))
 (via (at 30.0707 20.9) (size 0.6) (drill 0.3) (layers "F.Cu" "B.Cu") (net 3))
 (segment (start 30.0707 20.9) (end 28.0804 22.8903) (width 0.25) (layer "B.Cu") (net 3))
 (segment (start 28.0804 22.8903) (end 21.6054 22.8903) (width 0.25) (layer "B.Cu") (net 3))
 (segment (start 23.01 11.13) (end 23.01 11.942) (width 0.25) (layer "F.Cu") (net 5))
 (via (at 23.01 11.942) (size 0.6) (drill 0.3) (layers "F.Cu" "B.Cu") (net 5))
 (segment (start 24.6388 8.4068) (end 36.7182 8.4068) (width 0.25) (layer "B.Cu") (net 5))
 (segment (start 23.01 10.0356) (end 24.6388 8.4068) (width 0.25) (layer "B.Cu") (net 5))
 (segment (start 36.7182 8.4068) (end 37.705 7.42) (width 0.25) (layer "B.Cu") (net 5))
 (segment (start 23.01 11.942) (end 23.01 10.0356) (width 0.25) (layer "B.Cu") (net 5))
 (segment (start 30.3117 13.62) (end 32.6126 15.9209) (width 0.25) (layer "F.Cu") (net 13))
 (segment (start 30.3117 6.3975) (end 30.3117 13.62) (width 0.25) (layer "F.Cu") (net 13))
 (segment (start 0.8023 2.2925) (end 1.7314 2.2925) (width 0.25) (layer "F.Cu") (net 13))
 (segment (start 1.7314 2.2925) (end 1.7803 2.3414) (width 0.25) (layer "F.Cu") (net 13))
 (via (at 30.3117 6.3975) (size 0.6) (drill 0.3) (layers "F.Cu" "B.Cu") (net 13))
 (via (at 1.7803 2.3414) (size 0.6) (drill 0.3) (layers "F.Cu" "B.Cu") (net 13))
 (segment (start 30.3117 6.3975) (end 26.2556 2.3414) (width 0.25) (layer "B.Cu") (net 13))
 (segment (start 26.2556 2.3414) (end 1.7803 2.3414) (width 0.25) (layer "B.Cu") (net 13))
 (segment (start 17.643 9.86) (end 18.06 9.86) (width 0.25) (layer "F.Cu") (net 8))
 (segment (start 16.705 3.5415) (end 16.705 8.922) (width 0.25) (layer "F.Cu") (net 8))
 (segment (start 26.0881 11.1618) (end 26.0881 15.7573) (width 0.25) (layer "F.Cu") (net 8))
 (segment (start 22.0053 13.4217) (end 18.4436 9.86) (width 0.25) (layer "F.Cu") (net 8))
 (segment (start 16.705 8.922) (end 17.643 9.86) (width 0.25) (layer "F.Cu") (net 8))
 (segment (start 18.4436 9.86) (end 18.06 9.86) (width 0.25) (layer "F.Cu") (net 8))
 (segment (start 26.0881 15.7573) (end 22.4357 15.7573) (width 0.25) (layer "F.Cu") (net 8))
 (segment (start 19.4915 0.755) (end 16.705 3.5415) (width 0.25) (layer "F.Cu") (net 8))
 (segment (start 22.4357 15.7573) (end 22.0053 15.3269) (width 0.25) (layer "F.Cu") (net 8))
 (segment (start 22.0053 15.3269) (end 22.0053 13.4217) (width 0.25) (layer "F.Cu") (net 8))
 (segment (start 26.0881 15.7573) (end 26.0881 17.58) (width 0.25) (layer "F.Cu") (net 8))
 (segment (start 24.5406 0.755) (end 19.4915 0.755) (width 0.25) (layer "F.Cu") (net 8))
 (via (at 26.0881 17.58) (size 0.6) (drill 0.3) (layers "F.Cu" "B.Cu") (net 8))
 (segment (start 37.705 17.58) (end 26.0881 17.58) (width 0.25) (layer "B.Cu") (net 8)))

